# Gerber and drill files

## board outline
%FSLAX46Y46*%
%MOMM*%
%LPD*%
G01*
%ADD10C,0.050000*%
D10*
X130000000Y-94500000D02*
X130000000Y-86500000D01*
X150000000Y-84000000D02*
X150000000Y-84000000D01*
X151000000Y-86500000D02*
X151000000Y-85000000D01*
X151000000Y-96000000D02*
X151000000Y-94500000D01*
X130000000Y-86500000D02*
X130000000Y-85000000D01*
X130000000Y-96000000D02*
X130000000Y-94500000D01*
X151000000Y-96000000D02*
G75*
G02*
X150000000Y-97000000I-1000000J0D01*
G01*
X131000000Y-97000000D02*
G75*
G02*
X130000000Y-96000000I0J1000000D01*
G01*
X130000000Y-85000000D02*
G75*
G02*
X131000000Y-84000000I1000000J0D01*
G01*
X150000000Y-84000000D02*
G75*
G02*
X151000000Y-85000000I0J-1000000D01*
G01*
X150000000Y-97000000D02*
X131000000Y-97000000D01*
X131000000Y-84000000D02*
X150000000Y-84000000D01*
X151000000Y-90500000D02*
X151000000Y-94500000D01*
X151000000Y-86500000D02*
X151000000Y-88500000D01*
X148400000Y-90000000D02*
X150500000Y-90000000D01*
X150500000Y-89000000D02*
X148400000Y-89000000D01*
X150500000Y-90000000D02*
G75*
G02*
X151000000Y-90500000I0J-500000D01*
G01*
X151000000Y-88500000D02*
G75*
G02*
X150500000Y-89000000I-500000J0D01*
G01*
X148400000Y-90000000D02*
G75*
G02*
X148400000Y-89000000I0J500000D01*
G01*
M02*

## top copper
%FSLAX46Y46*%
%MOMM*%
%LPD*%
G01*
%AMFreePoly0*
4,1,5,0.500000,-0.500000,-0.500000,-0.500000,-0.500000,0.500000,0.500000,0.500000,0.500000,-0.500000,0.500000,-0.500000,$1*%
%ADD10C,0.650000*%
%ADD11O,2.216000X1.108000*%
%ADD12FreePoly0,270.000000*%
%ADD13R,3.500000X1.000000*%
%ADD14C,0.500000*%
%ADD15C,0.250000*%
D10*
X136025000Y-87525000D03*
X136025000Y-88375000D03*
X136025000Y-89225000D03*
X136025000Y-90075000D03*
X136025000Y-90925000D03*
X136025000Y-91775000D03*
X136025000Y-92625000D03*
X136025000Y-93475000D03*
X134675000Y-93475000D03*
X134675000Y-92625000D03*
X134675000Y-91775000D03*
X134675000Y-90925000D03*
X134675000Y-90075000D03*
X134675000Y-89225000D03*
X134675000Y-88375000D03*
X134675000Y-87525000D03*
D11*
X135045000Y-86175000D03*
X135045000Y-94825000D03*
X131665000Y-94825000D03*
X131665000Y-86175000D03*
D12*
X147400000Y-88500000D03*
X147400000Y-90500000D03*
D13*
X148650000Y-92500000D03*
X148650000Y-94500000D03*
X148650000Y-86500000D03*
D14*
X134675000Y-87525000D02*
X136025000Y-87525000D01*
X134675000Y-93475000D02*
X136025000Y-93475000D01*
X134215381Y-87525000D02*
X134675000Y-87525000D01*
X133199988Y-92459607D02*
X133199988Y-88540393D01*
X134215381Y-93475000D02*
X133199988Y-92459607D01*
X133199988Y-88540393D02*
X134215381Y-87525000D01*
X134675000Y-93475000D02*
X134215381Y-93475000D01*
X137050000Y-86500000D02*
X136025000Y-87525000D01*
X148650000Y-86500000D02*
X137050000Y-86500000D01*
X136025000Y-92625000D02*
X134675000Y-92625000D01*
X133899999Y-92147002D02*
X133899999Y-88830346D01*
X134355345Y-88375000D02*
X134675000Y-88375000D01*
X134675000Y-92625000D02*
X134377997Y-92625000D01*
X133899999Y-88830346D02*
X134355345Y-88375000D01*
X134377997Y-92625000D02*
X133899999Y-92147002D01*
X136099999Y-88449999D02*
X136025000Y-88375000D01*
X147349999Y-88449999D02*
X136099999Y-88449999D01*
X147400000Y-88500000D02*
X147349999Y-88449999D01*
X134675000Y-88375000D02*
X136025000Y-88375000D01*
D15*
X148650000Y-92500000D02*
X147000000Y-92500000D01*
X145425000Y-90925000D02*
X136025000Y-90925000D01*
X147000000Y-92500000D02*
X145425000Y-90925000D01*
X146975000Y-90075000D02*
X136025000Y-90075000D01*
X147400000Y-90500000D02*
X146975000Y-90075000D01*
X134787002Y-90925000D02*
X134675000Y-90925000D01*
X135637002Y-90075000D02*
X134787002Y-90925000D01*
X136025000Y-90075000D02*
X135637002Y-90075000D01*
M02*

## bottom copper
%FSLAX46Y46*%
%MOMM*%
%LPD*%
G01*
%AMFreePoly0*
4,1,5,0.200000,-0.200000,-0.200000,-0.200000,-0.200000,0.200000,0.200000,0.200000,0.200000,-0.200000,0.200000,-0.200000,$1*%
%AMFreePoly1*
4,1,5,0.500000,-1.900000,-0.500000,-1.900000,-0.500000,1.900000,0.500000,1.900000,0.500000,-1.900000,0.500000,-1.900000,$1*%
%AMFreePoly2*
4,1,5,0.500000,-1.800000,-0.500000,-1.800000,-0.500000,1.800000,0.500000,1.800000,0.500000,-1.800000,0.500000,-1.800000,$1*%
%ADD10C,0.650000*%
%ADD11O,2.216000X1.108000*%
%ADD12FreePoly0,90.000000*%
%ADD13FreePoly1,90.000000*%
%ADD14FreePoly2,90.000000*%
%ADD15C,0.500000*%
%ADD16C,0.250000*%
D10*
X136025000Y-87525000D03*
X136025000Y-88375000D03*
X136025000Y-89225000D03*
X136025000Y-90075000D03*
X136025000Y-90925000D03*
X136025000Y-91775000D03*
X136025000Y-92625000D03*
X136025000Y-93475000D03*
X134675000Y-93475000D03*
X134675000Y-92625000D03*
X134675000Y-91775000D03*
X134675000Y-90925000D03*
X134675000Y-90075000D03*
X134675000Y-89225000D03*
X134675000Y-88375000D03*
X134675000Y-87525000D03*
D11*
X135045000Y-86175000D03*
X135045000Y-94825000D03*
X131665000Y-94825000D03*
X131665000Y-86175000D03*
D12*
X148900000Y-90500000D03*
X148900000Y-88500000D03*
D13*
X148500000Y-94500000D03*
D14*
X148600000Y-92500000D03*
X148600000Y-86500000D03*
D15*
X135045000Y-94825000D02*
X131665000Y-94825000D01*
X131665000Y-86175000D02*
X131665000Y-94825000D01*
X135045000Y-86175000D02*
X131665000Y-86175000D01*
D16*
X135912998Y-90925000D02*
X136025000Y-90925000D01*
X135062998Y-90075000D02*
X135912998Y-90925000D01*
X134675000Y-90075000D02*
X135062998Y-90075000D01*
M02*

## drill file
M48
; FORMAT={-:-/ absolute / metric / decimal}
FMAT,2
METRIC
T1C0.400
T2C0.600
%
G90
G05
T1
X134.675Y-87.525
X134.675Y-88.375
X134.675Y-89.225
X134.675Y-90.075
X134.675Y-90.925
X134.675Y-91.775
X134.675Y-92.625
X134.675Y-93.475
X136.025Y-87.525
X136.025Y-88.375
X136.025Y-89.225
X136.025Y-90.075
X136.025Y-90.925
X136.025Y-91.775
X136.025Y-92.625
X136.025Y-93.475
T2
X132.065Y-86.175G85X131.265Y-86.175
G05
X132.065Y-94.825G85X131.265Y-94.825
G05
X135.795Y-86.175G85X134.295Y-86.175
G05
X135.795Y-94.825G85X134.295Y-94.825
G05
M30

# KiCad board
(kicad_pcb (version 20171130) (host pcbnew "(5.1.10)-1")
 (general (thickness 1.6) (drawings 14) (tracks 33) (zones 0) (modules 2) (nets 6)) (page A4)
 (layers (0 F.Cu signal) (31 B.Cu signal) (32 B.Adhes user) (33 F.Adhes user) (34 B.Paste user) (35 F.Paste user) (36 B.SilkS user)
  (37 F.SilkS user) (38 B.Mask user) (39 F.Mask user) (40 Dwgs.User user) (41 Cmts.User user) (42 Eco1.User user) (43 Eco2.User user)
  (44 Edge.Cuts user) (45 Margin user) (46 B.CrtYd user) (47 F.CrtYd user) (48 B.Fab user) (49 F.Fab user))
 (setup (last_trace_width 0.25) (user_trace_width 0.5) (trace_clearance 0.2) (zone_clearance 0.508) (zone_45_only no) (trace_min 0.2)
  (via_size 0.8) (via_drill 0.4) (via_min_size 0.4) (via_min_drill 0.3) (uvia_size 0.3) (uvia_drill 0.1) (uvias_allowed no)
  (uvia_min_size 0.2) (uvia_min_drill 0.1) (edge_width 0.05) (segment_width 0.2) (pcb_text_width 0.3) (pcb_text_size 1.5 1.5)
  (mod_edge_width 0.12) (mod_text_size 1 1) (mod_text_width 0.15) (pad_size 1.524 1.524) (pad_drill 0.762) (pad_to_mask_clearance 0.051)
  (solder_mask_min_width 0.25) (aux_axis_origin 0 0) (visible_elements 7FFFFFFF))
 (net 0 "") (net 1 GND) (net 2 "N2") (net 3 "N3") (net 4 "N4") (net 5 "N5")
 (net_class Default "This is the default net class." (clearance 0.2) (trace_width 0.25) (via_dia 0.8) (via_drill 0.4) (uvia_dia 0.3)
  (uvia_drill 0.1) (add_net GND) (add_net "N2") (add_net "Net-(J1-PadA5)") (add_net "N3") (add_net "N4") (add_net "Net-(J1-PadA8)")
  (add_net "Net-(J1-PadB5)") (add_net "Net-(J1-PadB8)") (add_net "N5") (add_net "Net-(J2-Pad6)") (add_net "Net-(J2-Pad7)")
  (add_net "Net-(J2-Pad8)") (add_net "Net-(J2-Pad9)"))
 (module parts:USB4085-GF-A (layer F.Cu) (at 132 90.5 270)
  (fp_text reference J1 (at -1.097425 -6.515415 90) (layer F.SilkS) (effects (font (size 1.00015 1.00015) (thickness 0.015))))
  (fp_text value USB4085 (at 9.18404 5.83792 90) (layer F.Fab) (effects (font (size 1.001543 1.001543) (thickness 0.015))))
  (pad A1 thru_hole circle (at -2.975 -4.025 270) (size 0.65 0.65) (drill 0.4) (layers *.Cu *.Mask) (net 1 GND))
  (pad A4 thru_hole circle (at -2.125 -4.025 270) (size 0.65 0.65) (drill 0.4) (layers *.Cu *.Mask) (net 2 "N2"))
  (pad A5 thru_hole circle (at -1.275 -4.025 270) (size 0.65 0.65) (drill 0.4) (layers *.Cu *.Mask))
  (pad A6 thru_hole circle (at -0.425 -4.025 270) (size 0.65 0.65) (drill 0.4) (layers *.Cu *.Mask) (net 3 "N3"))
  (pad A7 thru_hole circle (at 0.425 -4.025 270) (size 0.65 0.65) (drill 0.4) (layers *.Cu *.Mask) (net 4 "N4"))
  (pad A8 thru_hole circle (at 1.275 -4.025 270) (size 0.65 0.65) (drill 0.4) (layers *.Cu *.Mask))
  (pad A9 thru_hole circle (at 2.125 -4.025 270) (size 0.65 0.65) (drill 0.4) (layers *.Cu *.Mask) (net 2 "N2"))
  (pad A12 thru_hole circle (at 2.975 -4.025 270) (size 0.65 0.65) (drill 0.4) (layers *.Cu *.Mask) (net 1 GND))
  (pad B1 thru_hole circle (at 2.975 -2.675 270) (size 0.65 0.65) (drill 0.4) (layers *.Cu *.Mask) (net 1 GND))
  (pad B4 thru_hole circle (at 2.125 -2.675 270) (size 0.65 0.65) (drill 0.4) (layers *.Cu *.Mask) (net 2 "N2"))
  (pad B5 thru_hole circle (at 1.275 -2.675 270) (size 0.65 0.65) (drill 0.4) (layers *.Cu *.Mask))
  (pad B6 thru_hole circle (at 0.425 -2.675 270) (size 0.65 0.65) (drill 0.4) (layers *.Cu *.Mask) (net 3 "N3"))
  (pad B7 thru_hole circle (at -0.425 -2.675 270) (size 0.65 0.65) (drill 0.4) (layers *.Cu *.Mask) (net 4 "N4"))
  (pad B8 thru_hole circle (at -1.275 -2.675 270) (size 0.65 0.65) (drill 0.4) (layers *.Cu *.Mask))
  (pad B9 thru_hole circle (at -2.125 -2.675 270) (size 0.65 0.65) (drill 0.4) (layers *.Cu *.Mask) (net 2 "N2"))
  (pad B12 thru_hole circle (at -2.975 -2.675 270) (size 0.65 0.65) (drill 0.4) (layers *.Cu *.Mask) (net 1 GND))
  (pad P1 thru_hole oval (at -4.325 -3.045 270) (size 1.108 2.216) (drill oval 0.6 2.1) (layers *.Cu *.Mask) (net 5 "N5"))
  (pad P2 thru_hole oval (at 4.325 -3.045 270) (size 1.108 2.216) (drill oval 0.6 2.1) (layers *.Cu *.Mask) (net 5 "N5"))
  (pad P3 thru_hole oval (at 4.325 0.335 270) (size 1.108 2.216) (drill oval 0.6 1.4) (layers *.Cu *.Mask) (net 5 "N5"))
  (pad P4 thru_hole oval (at -4.325 0.335 270) (size 1.108 2.216) (drill oval 0.6 1.4) (layers *.Cu *.Mask) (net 5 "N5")))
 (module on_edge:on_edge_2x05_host (layer F.Cu) (at 151 90.5 270)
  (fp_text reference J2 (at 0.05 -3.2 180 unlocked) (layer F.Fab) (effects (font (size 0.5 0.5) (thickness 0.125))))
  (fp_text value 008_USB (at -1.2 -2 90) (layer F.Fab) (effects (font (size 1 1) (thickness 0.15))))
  (fp_line (start 0 0) (end 4 0) (layer Edge.Cuts) (width 0.05))
  (fp_line (start -4 0) (end -2 0) (layer Edge.Cuts) (width 0.05))
  (fp_line (start -0.5 2.6) (end -0.5 0.5) (layer Edge.Cuts) (width 0.05))
  (fp_line (start -1.5 0.5) (end -1.5 2.6) (layer Edge.Cuts) (width 0.05))
  (fp_arc (start 0 0.5) (end 0 0) (angle -90) (layer Edge.Cuts) (width 0.05))
  (fp_arc (start -2 0.5) (end -1.5 0.5) (angle -90) (layer Edge.Cuts) (width 0.05))
  (fp_arc (start -1 2.6) (end -1.5 2.6) (angle -180) (layer Edge.Cuts) (width 0.05))
  (pad 2 smd custom (at -2 3.6 270) (size 1 1) (layers F.Cu F.Mask) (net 2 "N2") (zone_connect 0)
   (options (clearance outline) (anchor rect)) (primitives))
  (pad 3 smd custom (at 0 3.6 270) (size 1 1) (layers F.Cu F.Mask) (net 3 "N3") (zone_connect 0) (options (clearance outline) (anchor rect))
   (primitives))
  (pad 8 smd custom (at 0 2.1 90) (size 0.4 0.4) (layers B.Cu B.Mask) (zone_connect 0) (options (clearance outline) (anchor rect))
   (primitives))
  (pad 7 smd custom (at -2 2.1 90) (size 0.4 0.4) (layers B.Cu B.Mask) (zone_connect 0) (options (clearance outline) (anchor rect))
   (primitives))
  (pad 4 smd rect (at 2 2.35 270) (size 1 3.5) (layers F.Cu F.Mask) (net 4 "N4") (zone_connect 0))
  (pad 10 smd custom (at 4 2.5 90) (size 1 3.8) (layers B.Cu B.Mask) (zone_connect 0) (options (clearance outline) (anchor rect))
   (primitives))
  (pad 9 smd custom (at 2 2.4 90) (size 1 3.6) (layers B.Cu B.Mask) (zone_connect 0) (options (clearance outline) (anchor rect))
   (primitives))
  (pad 6 smd custom (at -4 2.4 90) (size 1 3.6) (layers B.Cu B.Mask) (zone_connect 0) (options (clearance outline) (anchor rect))
   (primitives))
  (pad 5 smd rect (at 4 2.35 270) (size 1 3.5) (layers F.Cu F.Mask) (zone_connect 0))
  (pad 1 smd rect (at -4 2.35 270) (size 1 3.5) (layers F.Cu F.Mask) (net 1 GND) (zone_connect 0)))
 (gr_line (start 130 94.5) (end 130 86.5) (layer Edge.Cuts) (width 0.05))
 (gr_line (start 150 84) (end 150 84) (layer Edge.Cuts) (width 0.05))
 (gr_line (start 151 86.5) (end 151 85) (layer Edge.Cuts) (width 0.05))
 (gr_line (start 151 96) (end 151 94.5) (layer Edge.Cuts) (width 0.05))
 (gr_line (start 130 86.5) (end 130 85) (layer Edge.Cuts) (width 0.05))
 (gr_line (start 130 96) (end 130 94.5) (layer Edge.Cuts) (width 0.05))
 (gr_arc (start 150 96) (end 150 97) (angle -90) (layer Edge.Cuts) (width 0.05))
 (gr_arc (start 131 96) (end 130 96) (angle -90) (layer Edge.Cuts) (width 0.05))
 (gr_arc (start 131 85) (end 131 84) (angle -90) (layer Edge.Cuts) (width 0.05))
 (gr_arc (start 150 85) (end 151 85) (angle -90) (layer Edge.Cuts) (width 0.05))
 (gr_line (start 150 97) (end 131 97) (layer Edge.Cuts) (width 0.05))
 (gr_line (start 131 84) (end 150 84) (layer Edge.Cuts) (width 0.05))
 (segment (start 134.675 87.525) (end 136.025 87.525) (width 0.5) (layer F.Cu) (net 1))
 (segment (start 134.675 93.475) (end 136.025 93.475) (width 0.5) (layer F.Cu) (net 1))
 (segment (start 134.215381 87.525) (end 134.675 87.525) (width 0.5) (layer F.Cu) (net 1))
 (segment (start 133.199988 92.459607) (end 133.199988 88.540393) (width 0.5) (layer F.Cu) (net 1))
 (segment (start 134.215381 93.475) (end 133.199988 92.459607) (width 0.5) (layer F.Cu) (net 1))
 (segment (start 133.199988 88.540393) (end 134.215381 87.525) (width 0.5) (layer F.Cu) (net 1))
 (segment (start 134.675 93.475) (end 134.215381 93.475) (width 0.5) (layer F.Cu) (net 1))
 (segment (start 137.05 86.5) (end 136.025 87.525) (width 0.5) (layer F.Cu) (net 1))
 (segment (start 148.65 86.5) (end 137.05 86.5) (width 0.5) (layer F.Cu) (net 1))
 (segment (start 135.045 94.825) (end 131.665 94.825) (width 0.5) (layer B.Cu) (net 5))
 (segment (start 131.665 86.175) (end 131.665 94.825) (width 0.5) (layer B.Cu) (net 5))
 (segment (start 135.045 86.175) (end 131.665 86.175) (width 0.5) (layer B.Cu) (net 5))
 (segment (start 136.025 92.625) (end 134.675 92.625) (width 0.5) (layer F.Cu) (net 2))
 (segment (start 133.899999 92.147002) (end 133.899999 88.830346) (width 0.5) (layer F.Cu) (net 2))
 (segment (start 134.355345 88.375) (end 134.675 88.375) (width 0.5) (layer F.Cu) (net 2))
 (segment (start 134.675 92.625) (end 134.377997 92.625) (width 0.5) (layer F.Cu) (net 2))
 (segment (start 133.899999 88.830346) (end 134.355345 88.375) (width 0.5) (layer F.Cu) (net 2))
 (segment (start 134.377997 92.625) (end 133.899999 92.147002) (width 0.5) (layer F.Cu) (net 2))
 (segment (start 136.099999 88.449999) (end 136.025 88.375) (width 0.5) (layer F.Cu) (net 2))
 (segment (start 147.349999 88.449999) (end 136.099999 88.449999) (width 0.5) (layer F.Cu) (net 2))
 (segment (start 147.4 88.5) (end 147.349999 88.449999) (width 0.5) (layer F.Cu) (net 2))
 (segment (start 134.675 88.375) (end 136.025 88.375) (width 0.5) (layer F.Cu) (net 2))
 (segment (start 148.65 92.5) (end 147 92.5) (width 0.25) (layer F.Cu) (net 4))
 (segment (start 145.425 90.925) (end 136.025 90.925) (width 0.25) (layer F.Cu) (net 4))
 (segment (start 147 92.5) (end 145.425 90.925) (width 0.25) (layer F.Cu) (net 4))
 (segment (start 135.912998 90.925) (end 136.025 90.925) (width 0.25) (layer B.Cu) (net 4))
 (segment (start 135.062998 90.075) (end 135.912998 90.925) (width 0.25) (layer B.Cu) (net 4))
 (segment (start 134.675 90.075) (end 135.062998 90.075) (width 0.25) (layer B.Cu) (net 4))
 (segment (start 146.975 90.075) (end 136.025 90.075) (width 0.25) (layer F.Cu) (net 3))
 (segment (start 147.4 90.5) (end 146.975 90.075) (width 0.25) (layer F.Cu) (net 3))
 (segment (start 134.787002 90.925) (end 134.675 90.925) (width 0.25) (layer F.Cu) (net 3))
 (segment (start 135.637002 90.075) (end 134.787002 90.925) (width 0.25) (layer F.Cu) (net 3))
 (segment (start 136.025 90.075) (end 135.637002 90.075) (width 0.25) (layer F.Cu) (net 3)))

